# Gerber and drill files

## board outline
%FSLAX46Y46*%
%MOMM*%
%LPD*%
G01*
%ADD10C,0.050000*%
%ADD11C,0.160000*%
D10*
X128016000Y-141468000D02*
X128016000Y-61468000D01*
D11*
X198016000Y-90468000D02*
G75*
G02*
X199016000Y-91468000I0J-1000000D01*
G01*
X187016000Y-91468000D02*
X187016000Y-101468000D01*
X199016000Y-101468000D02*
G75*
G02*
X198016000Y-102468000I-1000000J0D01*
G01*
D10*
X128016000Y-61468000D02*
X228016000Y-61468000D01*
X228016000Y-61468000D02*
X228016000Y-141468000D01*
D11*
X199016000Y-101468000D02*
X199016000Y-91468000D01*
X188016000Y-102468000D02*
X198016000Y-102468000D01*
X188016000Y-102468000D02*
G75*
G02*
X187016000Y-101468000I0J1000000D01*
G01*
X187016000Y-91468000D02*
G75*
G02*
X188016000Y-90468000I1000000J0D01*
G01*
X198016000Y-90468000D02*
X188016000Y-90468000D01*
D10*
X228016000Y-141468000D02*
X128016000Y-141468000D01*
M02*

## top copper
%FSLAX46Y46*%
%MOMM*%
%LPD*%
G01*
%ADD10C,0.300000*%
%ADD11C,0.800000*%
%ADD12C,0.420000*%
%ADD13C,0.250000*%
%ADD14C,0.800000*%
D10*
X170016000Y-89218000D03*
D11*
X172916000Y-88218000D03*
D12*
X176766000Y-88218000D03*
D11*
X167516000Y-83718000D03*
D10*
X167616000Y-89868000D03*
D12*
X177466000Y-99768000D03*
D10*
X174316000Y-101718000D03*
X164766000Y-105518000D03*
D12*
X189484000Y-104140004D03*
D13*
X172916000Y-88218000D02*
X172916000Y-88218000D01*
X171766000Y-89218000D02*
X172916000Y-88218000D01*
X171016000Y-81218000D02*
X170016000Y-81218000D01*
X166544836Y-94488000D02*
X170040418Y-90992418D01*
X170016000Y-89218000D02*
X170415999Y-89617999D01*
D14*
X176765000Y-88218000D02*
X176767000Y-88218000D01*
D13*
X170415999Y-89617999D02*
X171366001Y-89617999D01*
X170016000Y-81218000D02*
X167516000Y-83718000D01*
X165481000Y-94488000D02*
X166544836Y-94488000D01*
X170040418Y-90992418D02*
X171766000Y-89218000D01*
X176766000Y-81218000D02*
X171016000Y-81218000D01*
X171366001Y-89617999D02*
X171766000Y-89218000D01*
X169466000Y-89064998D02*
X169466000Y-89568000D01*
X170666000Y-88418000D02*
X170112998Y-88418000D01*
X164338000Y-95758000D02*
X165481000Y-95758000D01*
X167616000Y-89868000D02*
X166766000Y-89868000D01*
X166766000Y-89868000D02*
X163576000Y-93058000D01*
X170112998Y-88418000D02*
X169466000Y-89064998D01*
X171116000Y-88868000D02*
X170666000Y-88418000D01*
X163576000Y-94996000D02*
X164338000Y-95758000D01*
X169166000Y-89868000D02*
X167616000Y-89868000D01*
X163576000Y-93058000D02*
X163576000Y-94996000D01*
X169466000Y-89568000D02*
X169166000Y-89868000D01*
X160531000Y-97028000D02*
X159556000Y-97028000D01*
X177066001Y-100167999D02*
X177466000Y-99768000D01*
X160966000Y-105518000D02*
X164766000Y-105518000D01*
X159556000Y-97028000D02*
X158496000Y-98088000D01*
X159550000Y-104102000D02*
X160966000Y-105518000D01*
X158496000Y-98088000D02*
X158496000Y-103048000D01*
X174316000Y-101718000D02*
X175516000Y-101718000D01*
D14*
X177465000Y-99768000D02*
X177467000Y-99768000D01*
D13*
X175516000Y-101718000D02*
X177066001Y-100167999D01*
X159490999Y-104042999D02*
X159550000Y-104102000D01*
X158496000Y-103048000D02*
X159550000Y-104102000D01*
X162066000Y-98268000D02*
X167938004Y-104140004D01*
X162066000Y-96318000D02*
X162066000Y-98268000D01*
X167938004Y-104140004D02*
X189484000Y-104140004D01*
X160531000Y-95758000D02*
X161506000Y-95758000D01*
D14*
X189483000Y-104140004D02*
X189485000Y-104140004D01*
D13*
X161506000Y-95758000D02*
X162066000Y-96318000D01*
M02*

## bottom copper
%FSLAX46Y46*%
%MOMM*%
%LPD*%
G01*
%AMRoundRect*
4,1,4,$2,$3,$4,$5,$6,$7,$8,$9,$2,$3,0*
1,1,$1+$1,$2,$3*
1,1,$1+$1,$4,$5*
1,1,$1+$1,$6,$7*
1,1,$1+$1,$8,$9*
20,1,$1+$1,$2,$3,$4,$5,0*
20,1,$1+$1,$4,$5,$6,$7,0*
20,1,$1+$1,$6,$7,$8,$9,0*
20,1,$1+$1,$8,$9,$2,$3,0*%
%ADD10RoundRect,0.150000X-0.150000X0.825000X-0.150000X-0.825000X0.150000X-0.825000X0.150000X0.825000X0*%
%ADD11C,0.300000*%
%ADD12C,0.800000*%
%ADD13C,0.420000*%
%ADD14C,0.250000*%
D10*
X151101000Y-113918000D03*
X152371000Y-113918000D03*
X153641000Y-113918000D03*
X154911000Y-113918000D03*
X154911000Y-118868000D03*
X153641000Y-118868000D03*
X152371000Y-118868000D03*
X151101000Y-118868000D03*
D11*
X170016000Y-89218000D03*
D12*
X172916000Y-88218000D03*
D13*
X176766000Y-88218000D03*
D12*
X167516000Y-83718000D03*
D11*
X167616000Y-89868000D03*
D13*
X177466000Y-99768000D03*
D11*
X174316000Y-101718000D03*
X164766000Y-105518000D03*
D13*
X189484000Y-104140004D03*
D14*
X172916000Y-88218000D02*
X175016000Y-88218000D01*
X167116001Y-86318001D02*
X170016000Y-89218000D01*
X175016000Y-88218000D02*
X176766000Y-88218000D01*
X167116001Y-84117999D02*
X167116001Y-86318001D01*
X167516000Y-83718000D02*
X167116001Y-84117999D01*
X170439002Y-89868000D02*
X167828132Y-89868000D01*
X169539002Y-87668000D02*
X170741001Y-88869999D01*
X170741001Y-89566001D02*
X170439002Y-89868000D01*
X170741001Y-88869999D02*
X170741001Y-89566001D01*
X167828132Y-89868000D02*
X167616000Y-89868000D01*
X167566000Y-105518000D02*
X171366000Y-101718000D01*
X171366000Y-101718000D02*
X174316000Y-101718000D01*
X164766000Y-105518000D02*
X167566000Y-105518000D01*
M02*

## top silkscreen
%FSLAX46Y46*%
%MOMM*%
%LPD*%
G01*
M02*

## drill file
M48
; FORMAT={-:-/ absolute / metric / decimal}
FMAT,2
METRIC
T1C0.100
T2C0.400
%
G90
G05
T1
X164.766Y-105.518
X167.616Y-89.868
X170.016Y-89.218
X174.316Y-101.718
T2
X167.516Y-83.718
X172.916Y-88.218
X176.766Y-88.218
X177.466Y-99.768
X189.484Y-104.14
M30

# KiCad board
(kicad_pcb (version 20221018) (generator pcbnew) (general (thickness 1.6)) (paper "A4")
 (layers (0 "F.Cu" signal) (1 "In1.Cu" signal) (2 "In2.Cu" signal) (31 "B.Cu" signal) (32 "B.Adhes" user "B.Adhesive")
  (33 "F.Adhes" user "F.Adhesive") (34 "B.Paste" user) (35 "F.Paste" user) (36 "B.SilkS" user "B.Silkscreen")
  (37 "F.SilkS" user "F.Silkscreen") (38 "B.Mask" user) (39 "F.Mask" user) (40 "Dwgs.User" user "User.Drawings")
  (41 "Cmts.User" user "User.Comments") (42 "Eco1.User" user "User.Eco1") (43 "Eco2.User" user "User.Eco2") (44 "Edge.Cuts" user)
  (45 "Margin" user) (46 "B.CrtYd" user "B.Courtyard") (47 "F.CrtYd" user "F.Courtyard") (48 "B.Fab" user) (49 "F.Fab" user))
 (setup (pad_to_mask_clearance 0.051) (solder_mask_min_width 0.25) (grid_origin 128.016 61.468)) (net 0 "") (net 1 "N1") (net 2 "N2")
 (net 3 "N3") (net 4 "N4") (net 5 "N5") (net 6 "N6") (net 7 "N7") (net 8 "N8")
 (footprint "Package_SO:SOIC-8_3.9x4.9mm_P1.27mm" (layer "B.Cu") (at 153.006 116.393 -90)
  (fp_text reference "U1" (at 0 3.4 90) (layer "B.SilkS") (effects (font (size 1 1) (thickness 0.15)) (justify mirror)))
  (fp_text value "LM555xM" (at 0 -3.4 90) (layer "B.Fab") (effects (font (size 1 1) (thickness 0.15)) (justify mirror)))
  (pad "1" smd roundrect (at -2.475 1.905 270) (size 1.95 0.6) (layers "B.Cu" "B.Paste" "B.Mask") (roundrect_rratio 0.25) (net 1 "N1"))
  (pad "2" smd roundrect (at -2.475 0.635 270) (size 1.95 0.6) (layers "B.Cu" "B.Paste" "B.Mask") (roundrect_rratio 0.25) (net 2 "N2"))
  (pad "3" smd roundrect (at -2.475 -0.635 270) (size 1.95 0.6) (layers "B.Cu" "B.Paste" "B.Mask") (roundrect_rratio 0.25) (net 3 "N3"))
  (pad "4" smd roundrect (at -2.475 -1.905 270) (size 1.95 0.6) (layers "B.Cu" "B.Paste" "B.Mask") (roundrect_rratio 0.25) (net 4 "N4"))
  (pad "5" smd roundrect (at 2.475 -1.905 270) (size 1.95 0.6) (layers "B.Cu" "B.Paste" "B.Mask") (roundrect_rratio 0.25) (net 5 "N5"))
  (pad "6" smd roundrect (at 2.475 -0.635 270) (size 1.95 0.6) (layers "B.Cu" "B.Paste" "B.Mask") (roundrect_rratio 0.25) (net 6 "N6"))
  (pad "7" smd roundrect (at 2.475 0.635 270) (size 1.95 0.6) (layers "B.Cu" "B.Paste" "B.Mask") (roundrect_rratio 0.25) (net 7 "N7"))
  (pad "8" smd roundrect (at 2.475 1.905 270) (size 1.95 0.6) (layers "B.Cu" "B.Paste" "B.Mask") (roundrect_rratio 0.25) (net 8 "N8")))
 (gr_line (start 128.016 141.468) (end 128.016 61.468) (stroke (width 0.05) (type solid)) (layer "Edge.Cuts"))
 (gr_arc (start 198.016 90.468) (mid 198.723107 90.760893) (end 199.016 91.468) (stroke (width 0.16) (type solid)) (layer "Edge.Cuts"))
 (gr_line (start 187.016 91.468) (end 187.016 101.468) (stroke (width 0.16) (type solid)) (layer "Edge.Cuts"))
 (gr_arc (start 199.016 101.468) (mid 198.723107 102.175107) (end 198.016 102.468) (stroke (width 0.16) (type solid)) (layer "Edge.Cuts"))
 (gr_line (start 128.016 61.468) (end 228.016 61.468) (stroke (width 0.05) (type solid)) (layer "Edge.Cuts"))
 (gr_line (start 228.016 61.468) (end 228.016 141.468) (stroke (width 0.05) (type solid)) (layer "Edge.Cuts"))
 (gr_line (start 199.016 101.468) (end 199.016 91.468) (stroke (width 0.16) (type solid)) (layer "Edge.Cuts"))
 (gr_line (start 188.016 102.468) (end 198.016 102.468) (stroke (width 0.16) (type solid)) (layer "Edge.Cuts"))
 (gr_arc (start 188.016 102.468) (mid 187.308893 102.175107) (end 187.016 101.468) (stroke (width 0.16) (type solid)) (layer "Edge.Cuts"))
 (gr_arc (start 187.016 91.468) (mid 187.308893 90.760893) (end 188.016 90.468) (stroke (width 0.16) (type solid)) (layer "Edge.Cuts"))
 (gr_line (start 198.016 90.468) (end 188.016 90.468) (stroke (width 0.16) (type solid)) (layer "Edge.Cuts"))
 (gr_line (start 228.016 141.468) (end 128.016 141.468) (stroke (width 0.05) (type solid)) (layer "Edge.Cuts"))
 (segment (start 172.916 88.218) (end 172.916 88.218) (width 0.25) (layer "F.Cu") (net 8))
 (segment (start 171.766 89.218) (end 172.916 88.218) (width 0.25) (layer "F.Cu") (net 8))
 (segment (start 171.016 81.218) (end 170.016 81.218) (width 0.25) (layer "F.Cu") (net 8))
 (segment (start 166.544836 94.488) (end 170.040418 90.992418) (width 0.25) (layer "F.Cu") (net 8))
 (segment (start 170.016 89.218) (end 170.415999 89.617999) (width 0.25) (layer "F.Cu") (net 8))
 (segment (start 176.765 88.218) (end 176.767 88.218) (width 0.8) (layer "F.Cu") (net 8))
 (segment (start 170.415999 89.617999) (end 171.366001 89.617999) (width 0.25) (layer "F.Cu") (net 8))
 (segment (start 170.016 81.218) (end 167.516 83.718) (width 0.25) (layer "F.Cu") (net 8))
 (segment (start 165.481 94.488) (end 166.544836 94.488) (width 0.25) (layer "F.Cu") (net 8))
 (segment (start 170.040418 90.992418) (end 171.766 89.218) (width 0.25) (layer "F.Cu") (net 8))
 (segment (start 176.766 81.218) (end 171.016 81.218) (width 0.25) (layer "F.Cu") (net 8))
 (segment (start 171.366001 89.617999) (end 171.766 89.218) (width 0.25) (layer "F.Cu") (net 8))
 (via (at 170.016 89.218) (size 0.3) (drill 0.1) (layers "F.Cu" "B.Cu") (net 8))
 (via (at 172.916 88.218) (size 0.8) (drill 0.4) (layers "F.Cu" "B.Cu") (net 8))
 (via (at 176.766 88.218) (size 0.42) (drill 0.4) (layers "F.Cu" "B.Cu") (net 8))
 (via (at 167.516 83.718) (size 0.8) (drill 0.4) (layers "F.Cu" "B.Cu") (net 8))
 (segment (start 172.916 88.218) (end 175.016 88.218) (width 0.25) (layer "B.Cu") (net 8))
 (segment (start 167.116001 86.318001) (end 170.016 89.218) (width 0.25) (layer "B.Cu") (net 8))
 (segment (start 175.016 88.218) (end 176.766 88.218) (width 0.25) (layer "B.Cu") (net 8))
 (segment (start 167.116001 84.117999) (end 167.116001 86.318001) (width 0.25) (layer "B.Cu") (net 8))
 (segment (start 167.516 83.718) (end 167.116001 84.117999) (width 0.25) (layer "B.Cu") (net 8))
 (segment (start 169.466 89.064998) (end 169.466 89.568) (width 0.25) (layer "F.Cu") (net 7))
 (segment (start 170.666 88.418) (end 170.112998 88.418) (width 0.25) (layer "F.Cu") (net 7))
 (segment (start 164.338 95.758) (end 165.481 95.758) (width 0.25) (layer "F.Cu") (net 7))
 (segment (start 167.616 89.868) (end 166.766 89.868) (width 0.25) (layer "F.Cu") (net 7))
 (segment (start 166.766 89.868) (end 163.576 93.058) (width 0.25) (layer "F.Cu") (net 7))
 (segment (start 170.112998 88.418) (end 169.466 89.064998) (width 0.25) (layer "F.Cu") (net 7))
 (segment (start 171.116 88.868) (end 170.666 88.418) (width 0.25) (layer "F.Cu") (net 7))
 (segment (start 163.576 94.996) (end 164.338 95.758) (width 0.25) (layer "F.Cu") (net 7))
 (segment (start 169.166 89.868) (end 167.616 89.868) (width 0.25) (layer "F.Cu") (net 7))
 (segment (start 163.576 93.058) (end 163.576 94.996) (width 0.25) (layer "F.Cu") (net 7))
 (segment (start 169.466 89.568) (end 169.166 89.868) (width 0.25) (layer "F.Cu") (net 7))
 (via (at 167.616 89.868) (size 0.3) (drill 0.1) (layers "F.Cu" "B.Cu") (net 7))
 (segment (start 170.439002 89.868) (end 167.828132 89.868) (width 0.25) (layer "B.Cu") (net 7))
 (segment (start 169.539002 87.668) (end 170.741001 88.869999) (width 0.25) (layer "B.Cu") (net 7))
 (segment (start 170.741001 89.566001) (end 170.439002 89.868) (width 0.25) (layer "B.Cu") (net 7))
 (segment (start 170.741001 88.869999) (end 170.741001 89.566001) (width 0.25) (layer "B.Cu") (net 7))
 (segment (start 167.828132 89.868) (end 167.616 89.868) (width 0.25) (layer "B.Cu") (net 7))
 (segment (start 160.531 97.028) (end 159.556 97.028) (width 0.25) (layer "F.Cu") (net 3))
 (segment (start 177.066001 100.167999) (end 177.466 99.768) (width 0.25) (layer "F.Cu") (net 3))
 (segment (start 160.966 105.518) (end 164.766 105.518) (width 0.25) (layer "F.Cu") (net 3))
 (segment (start 159.556 97.028) (end 158.496 98.088) (width 0.25) (layer "F.Cu") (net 3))
 (segment (start 159.55 104.102) (end 160.966 105.518) (width 0.25) (layer "F.Cu") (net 3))
 (segment (start 158.496 98.088) (end 158.496 103.048) (width 0.25) (layer "F.Cu") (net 3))
 (segment (start 174.316 101.718) (end 175.516 101.718) (width 0.25) (layer "F.Cu") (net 3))
 (segment (start 177.465 99.768) (end 177.467 99.768) (width 0.8) (layer "F.Cu") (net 3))
 (segment (start 175.516 101.718) (end 177.066001 100.167999) (width 0.25) (layer "F.Cu") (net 3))
 (segment (start 159.490999 104.042999) (end 159.55 104.102) (width 0.25) (layer "F.Cu") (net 3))
 (segment (start 158.496 103.048) (end 159.55 104.102) (width 0.25) (layer "F.Cu") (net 3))
 (via (at 177.466 99.768) (size 0.42) (drill 0.4) (layers "F.Cu" "B.Cu") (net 3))
 (via (at 174.316 101.718) (size 0.3) (drill 0.1) (layers "F.Cu" "B.Cu") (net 3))
 (via (at 164.766 105.518) (size 0.3) (drill 0.1) (layers "F.Cu" "B.Cu") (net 3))
 (segment (start 167.566 105.518) (end 171.366 101.718) (width 0.25) (layer "B.Cu") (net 3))
 (segment (start 171.366 101.718) (end 174.316 101.718) (width 0.25) (layer "B.Cu") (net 3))
 (segment (start 164.766 105.518) (end 167.566 105.518) (width 0.25) (layer "B.Cu") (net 3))
 (segment (start 162.066 98.268) (end 167.938004 104.140004) (width 0.25) (layer "F.Cu") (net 2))
 (segment (start 162.066 96.318) (end 162.066 98.268) (width 0.25) (layer "F.Cu") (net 2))
 (segment (start 167.938004 104.140004) (end 189.484 104.140004) (width 0.25) (layer "F.Cu") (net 2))
 (segment (start 160.531 95.758) (end 161.506 95.758) (width 0.25) (layer "F.Cu") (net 2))
 (segment (start 189.483 104.140004) (end 189.485 104.140004) (width 0.8) (layer "F.Cu") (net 2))
 (segment (start 161.506 95.758) (end 162.066 96.318) (width 0.25) (layer "F.Cu") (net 2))
 (via (at 189.484 104.140004) (size 0.42) (drill 0.4) (layers "F.Cu" "B.Cu") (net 2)))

